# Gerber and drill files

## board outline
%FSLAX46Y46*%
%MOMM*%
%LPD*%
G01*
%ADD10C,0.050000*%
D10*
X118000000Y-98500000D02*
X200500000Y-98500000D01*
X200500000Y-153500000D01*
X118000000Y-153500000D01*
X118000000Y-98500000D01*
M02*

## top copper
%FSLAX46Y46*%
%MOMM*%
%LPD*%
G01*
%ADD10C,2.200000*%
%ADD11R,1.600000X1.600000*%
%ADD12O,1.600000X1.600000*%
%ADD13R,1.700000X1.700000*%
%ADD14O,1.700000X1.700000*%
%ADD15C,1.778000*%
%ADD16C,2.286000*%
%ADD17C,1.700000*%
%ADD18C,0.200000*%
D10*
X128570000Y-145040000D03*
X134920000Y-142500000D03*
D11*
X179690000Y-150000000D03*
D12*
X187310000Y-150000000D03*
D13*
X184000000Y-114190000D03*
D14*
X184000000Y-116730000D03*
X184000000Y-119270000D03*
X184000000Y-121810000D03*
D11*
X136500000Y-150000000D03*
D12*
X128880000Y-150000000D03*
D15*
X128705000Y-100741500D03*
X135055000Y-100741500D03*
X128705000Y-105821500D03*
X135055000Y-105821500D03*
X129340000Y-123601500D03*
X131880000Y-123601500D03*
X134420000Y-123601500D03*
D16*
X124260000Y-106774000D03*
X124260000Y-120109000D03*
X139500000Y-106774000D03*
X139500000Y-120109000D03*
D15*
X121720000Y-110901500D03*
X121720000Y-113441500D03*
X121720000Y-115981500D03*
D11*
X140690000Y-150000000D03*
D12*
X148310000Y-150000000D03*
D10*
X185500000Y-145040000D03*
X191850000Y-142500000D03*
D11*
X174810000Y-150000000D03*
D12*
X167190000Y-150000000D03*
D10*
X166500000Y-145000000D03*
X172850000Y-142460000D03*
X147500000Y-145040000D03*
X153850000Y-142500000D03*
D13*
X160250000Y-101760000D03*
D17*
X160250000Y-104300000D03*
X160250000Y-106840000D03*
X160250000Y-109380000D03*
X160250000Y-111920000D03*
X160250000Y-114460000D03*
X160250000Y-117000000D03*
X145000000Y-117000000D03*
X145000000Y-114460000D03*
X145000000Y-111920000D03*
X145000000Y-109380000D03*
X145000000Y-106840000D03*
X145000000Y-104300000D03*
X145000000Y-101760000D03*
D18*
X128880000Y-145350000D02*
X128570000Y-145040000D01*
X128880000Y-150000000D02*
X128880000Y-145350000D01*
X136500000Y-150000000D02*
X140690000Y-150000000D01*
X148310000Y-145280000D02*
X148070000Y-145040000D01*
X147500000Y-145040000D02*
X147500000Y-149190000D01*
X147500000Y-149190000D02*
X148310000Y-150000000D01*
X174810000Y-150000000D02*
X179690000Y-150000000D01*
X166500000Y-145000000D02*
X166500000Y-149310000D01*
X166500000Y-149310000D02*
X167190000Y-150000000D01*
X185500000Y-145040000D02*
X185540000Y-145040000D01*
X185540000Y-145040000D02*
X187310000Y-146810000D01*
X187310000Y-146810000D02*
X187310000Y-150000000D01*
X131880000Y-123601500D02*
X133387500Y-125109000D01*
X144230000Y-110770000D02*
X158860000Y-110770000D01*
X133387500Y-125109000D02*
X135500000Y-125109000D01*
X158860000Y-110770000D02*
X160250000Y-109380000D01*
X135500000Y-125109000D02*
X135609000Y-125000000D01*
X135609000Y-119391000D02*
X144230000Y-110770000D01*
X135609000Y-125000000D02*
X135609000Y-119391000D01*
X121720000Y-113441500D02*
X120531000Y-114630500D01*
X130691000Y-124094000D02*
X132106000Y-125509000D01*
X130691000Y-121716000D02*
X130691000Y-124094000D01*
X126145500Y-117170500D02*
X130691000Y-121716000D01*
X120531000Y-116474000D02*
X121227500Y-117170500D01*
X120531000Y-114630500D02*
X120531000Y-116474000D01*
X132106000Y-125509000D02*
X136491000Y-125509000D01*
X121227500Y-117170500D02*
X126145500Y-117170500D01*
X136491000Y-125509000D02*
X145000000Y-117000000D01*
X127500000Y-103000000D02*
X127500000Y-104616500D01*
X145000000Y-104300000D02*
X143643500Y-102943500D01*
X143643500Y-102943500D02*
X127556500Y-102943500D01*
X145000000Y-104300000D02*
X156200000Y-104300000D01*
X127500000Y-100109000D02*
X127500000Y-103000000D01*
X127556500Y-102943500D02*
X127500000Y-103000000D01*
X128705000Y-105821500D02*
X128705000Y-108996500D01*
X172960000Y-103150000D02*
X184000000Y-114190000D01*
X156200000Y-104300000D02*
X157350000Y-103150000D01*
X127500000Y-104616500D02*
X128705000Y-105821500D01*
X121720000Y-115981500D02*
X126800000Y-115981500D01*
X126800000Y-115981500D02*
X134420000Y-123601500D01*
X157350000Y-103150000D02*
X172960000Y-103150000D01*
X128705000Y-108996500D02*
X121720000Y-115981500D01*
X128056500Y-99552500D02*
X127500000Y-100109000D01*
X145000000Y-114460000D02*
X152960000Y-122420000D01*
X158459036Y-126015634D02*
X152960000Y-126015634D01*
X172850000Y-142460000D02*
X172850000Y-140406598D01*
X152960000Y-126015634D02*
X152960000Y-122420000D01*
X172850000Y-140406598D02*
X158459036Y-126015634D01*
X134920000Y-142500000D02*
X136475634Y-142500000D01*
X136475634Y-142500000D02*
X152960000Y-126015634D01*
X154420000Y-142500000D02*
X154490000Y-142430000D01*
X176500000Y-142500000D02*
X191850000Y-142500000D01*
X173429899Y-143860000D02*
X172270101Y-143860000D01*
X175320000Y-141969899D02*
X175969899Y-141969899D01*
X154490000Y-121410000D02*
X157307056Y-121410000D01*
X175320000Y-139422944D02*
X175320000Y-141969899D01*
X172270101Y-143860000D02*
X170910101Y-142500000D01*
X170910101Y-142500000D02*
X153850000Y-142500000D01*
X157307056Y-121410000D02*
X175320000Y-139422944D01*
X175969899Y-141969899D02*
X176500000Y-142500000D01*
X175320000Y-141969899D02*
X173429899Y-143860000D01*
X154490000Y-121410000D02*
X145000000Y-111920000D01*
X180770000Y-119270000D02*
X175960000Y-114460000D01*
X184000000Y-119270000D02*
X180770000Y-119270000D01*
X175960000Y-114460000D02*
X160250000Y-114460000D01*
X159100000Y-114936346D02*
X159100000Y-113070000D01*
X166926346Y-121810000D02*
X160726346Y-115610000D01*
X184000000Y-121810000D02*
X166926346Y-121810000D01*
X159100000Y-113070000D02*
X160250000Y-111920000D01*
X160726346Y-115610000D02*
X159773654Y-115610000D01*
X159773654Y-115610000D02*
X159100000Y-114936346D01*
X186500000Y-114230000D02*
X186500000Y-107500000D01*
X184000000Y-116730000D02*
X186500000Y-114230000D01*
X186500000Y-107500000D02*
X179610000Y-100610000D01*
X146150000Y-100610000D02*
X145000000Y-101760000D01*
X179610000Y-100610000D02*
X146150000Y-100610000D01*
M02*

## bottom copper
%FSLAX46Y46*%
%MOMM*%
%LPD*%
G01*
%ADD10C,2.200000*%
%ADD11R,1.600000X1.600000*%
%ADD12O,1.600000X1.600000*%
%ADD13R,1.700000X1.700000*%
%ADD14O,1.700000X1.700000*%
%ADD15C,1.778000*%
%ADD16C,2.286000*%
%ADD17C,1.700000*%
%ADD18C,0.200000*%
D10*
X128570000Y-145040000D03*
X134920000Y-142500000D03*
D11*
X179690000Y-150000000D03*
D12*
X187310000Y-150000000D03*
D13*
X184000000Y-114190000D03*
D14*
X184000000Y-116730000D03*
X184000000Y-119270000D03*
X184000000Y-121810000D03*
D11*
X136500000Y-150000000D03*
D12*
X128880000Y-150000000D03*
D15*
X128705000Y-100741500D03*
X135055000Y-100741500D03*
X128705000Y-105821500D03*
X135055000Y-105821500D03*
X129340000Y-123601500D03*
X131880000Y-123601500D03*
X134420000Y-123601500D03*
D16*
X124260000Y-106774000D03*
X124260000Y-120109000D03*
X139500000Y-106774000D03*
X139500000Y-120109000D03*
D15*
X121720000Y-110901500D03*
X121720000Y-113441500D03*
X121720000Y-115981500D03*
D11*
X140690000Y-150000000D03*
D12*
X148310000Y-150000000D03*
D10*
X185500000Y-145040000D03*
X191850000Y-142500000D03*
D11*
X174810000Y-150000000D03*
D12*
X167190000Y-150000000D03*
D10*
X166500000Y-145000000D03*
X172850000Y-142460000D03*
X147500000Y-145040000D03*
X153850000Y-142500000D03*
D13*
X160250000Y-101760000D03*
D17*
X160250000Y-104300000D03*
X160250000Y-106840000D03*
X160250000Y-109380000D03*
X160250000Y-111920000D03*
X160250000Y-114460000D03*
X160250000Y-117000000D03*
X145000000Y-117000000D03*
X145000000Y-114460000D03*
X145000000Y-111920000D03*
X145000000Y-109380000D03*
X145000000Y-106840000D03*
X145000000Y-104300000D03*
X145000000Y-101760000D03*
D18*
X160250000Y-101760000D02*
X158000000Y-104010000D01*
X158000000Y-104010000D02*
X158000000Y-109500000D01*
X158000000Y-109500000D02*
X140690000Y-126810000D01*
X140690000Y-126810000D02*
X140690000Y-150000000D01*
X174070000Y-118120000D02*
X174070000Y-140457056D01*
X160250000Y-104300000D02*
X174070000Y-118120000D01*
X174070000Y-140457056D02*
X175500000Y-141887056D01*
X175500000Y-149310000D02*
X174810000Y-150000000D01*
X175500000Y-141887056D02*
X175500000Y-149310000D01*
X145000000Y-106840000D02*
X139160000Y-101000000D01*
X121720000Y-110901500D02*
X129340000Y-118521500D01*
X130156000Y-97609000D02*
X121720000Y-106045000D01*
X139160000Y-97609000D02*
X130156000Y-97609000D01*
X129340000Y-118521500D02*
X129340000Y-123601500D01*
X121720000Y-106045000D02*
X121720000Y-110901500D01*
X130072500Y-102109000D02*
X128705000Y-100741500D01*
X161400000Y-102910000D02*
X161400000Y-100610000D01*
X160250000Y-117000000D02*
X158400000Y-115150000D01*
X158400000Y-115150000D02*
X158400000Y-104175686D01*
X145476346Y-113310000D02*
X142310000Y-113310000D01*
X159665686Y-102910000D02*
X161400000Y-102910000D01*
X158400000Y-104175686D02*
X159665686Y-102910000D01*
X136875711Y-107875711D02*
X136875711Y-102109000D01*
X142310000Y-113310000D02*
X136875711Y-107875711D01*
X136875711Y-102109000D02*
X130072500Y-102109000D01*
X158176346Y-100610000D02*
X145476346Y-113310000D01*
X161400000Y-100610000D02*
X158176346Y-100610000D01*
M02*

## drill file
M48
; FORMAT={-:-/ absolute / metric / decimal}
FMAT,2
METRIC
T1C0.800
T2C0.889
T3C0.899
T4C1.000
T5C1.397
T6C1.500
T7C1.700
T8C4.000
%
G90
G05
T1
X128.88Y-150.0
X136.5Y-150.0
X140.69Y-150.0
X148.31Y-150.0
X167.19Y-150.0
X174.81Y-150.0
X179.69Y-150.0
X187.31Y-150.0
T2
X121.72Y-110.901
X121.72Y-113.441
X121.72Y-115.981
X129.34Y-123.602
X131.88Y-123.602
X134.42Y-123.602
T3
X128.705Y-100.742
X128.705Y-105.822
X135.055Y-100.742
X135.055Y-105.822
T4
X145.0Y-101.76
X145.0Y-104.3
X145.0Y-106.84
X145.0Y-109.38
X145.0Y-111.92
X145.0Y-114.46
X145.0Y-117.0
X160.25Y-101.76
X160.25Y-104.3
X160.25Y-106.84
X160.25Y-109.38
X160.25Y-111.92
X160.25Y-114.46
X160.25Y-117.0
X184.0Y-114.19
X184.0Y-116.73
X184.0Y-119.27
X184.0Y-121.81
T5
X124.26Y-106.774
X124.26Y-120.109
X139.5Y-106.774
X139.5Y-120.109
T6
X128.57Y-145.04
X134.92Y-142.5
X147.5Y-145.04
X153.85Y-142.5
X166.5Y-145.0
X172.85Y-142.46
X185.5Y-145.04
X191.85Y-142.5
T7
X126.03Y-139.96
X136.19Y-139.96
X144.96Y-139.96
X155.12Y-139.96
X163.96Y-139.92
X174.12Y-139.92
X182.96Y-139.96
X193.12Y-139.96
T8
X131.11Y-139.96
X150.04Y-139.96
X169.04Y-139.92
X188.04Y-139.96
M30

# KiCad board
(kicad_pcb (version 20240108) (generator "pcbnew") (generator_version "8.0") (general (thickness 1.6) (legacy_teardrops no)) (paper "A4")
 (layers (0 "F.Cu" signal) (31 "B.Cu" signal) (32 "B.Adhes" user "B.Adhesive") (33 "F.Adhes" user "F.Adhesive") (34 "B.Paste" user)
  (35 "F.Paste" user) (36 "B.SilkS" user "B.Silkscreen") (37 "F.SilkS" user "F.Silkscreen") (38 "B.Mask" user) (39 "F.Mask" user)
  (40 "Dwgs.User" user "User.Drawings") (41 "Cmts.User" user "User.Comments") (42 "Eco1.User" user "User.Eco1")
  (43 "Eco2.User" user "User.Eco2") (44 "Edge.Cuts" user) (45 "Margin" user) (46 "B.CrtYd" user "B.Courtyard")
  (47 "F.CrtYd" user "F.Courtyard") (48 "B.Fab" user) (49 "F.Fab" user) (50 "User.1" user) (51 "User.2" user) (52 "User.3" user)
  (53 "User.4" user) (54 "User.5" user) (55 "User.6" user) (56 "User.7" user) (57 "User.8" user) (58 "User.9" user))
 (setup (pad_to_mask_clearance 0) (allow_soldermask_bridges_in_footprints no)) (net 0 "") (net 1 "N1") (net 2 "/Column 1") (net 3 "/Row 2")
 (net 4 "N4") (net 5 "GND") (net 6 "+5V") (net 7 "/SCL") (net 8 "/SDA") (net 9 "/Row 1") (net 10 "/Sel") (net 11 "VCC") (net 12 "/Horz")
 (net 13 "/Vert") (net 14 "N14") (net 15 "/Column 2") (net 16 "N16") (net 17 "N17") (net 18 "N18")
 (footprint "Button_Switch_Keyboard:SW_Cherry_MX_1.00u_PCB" (layer "F.Cu") (at 128.57 145.04 180)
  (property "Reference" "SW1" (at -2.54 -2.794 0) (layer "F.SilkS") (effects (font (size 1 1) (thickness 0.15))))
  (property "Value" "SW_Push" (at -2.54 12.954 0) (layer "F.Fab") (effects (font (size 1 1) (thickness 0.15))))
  (pad "" np_thru_hole circle (at -7.62 5.08 180) (size 1.7 1.7) (drill 1.7) (layers "*.Cu" "*.Mask"))
  (pad "" np_thru_hole circle (at -2.54 5.08 180) (size 4 4) (drill 4) (layers "*.Cu" "*.Mask"))
  (pad "" np_thru_hole circle (at 2.54 5.08 180) (size 1.7 1.7) (drill 1.7) (layers "*.Cu" "*.Mask"))
  (pad "1" thru_hole circle (at 0 0 180) (size 2.2 2.2) (drill 1.5) (layers "*.Cu" "*.Mask") (remove_unused_layers no) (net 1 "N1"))
  (pad "2" thru_hole circle (at -6.35 2.54 180) (size 2.2 2.2) (drill 1.5) (layers "*.Cu" "*.Mask") (remove_unused_layers no)
   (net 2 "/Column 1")))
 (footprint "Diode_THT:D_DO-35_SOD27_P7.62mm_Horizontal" (layer "F.Cu") (at 179.69 150)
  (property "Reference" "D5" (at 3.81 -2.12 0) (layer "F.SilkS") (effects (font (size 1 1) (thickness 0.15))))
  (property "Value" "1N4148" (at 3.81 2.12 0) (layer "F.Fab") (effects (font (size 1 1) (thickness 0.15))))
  (pad "1" thru_hole rect (at 0 0) (size 1.6 1.6) (drill 0.8) (layers "*.Cu" "*.Mask") (remove_unused_layers no) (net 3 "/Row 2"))
  (pad "2" thru_hole oval (at 7.62 0) (size 1.6 1.6) (drill 0.8) (layers "*.Cu" "*.Mask") (remove_unused_layers no) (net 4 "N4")))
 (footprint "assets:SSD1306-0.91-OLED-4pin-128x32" (layer "F.Cu") (at 147.5 112)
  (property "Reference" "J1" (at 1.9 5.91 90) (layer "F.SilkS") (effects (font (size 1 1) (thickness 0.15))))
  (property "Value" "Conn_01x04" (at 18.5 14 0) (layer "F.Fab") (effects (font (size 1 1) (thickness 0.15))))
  (pad "1" thru_hole rect (at 36.5 2.19) (size 1.7 1.7) (drill 1) (layers "*.Cu" "*.Mask") (remove_unused_layers no) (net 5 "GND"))
  (pad "2" thru_hole oval (at 36.5 4.73) (size 1.7 1.7) (drill 1) (layers "*.Cu" "*.Mask") (remove_unused_layers no) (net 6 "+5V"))
  (pad "3" thru_hole oval (at 36.5 7.27) (size 1.7 1.7) (drill 1) (layers "*.Cu" "*.Mask") (remove_unused_layers no) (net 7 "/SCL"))
  (pad "4" thru_hole oval (at 36.5 9.81) (size 1.7 1.7) (drill 1) (layers "*.Cu" "*.Mask") (remove_unused_layers no) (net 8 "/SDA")))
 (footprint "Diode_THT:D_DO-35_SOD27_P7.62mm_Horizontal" (layer "F.Cu") (at 136.5 150 180)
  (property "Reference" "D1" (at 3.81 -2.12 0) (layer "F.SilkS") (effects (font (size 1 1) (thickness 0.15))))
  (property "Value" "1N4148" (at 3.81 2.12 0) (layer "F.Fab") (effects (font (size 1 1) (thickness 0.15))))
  (pad "1" thru_hole rect (at 0 0 180) (size 1.6 1.6) (drill 0.8) (layers "*.Cu" "*.Mask") (remove_unused_layers no) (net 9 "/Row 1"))
  (pad "2" thru_hole oval (at 7.62 0 180) (size 1.6 1.6) (drill 0.8) (layers "*.Cu" "*.Mask") (remove_unused_layers no) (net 1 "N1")))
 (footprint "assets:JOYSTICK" (layer "F.Cu") (at 131.88 113.4415)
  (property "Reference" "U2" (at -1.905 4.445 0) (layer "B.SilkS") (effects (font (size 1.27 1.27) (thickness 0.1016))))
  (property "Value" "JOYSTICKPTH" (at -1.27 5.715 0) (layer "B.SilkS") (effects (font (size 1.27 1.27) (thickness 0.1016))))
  (pad "B1A" thru_hole circle (at -3.175 -12.7) (size 1.778 1.778) (drill 0.89916) (layers "F&B.Cu" "F.Paste" "F.SilkS" "F.Mask")
   (remove_unused_layers no) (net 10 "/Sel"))
  (pad "B1B" thru_hole circle (at 3.175 -12.7) (size 1.778 1.778) (drill 0.89916) (layers "F&B.Cu" "F.Paste" "F.SilkS" "F.Mask")
   (remove_unused_layers no))
  (pad "B2A" thru_hole circle (at -3.175 -7.62) (size 1.778 1.778) (drill 0.89916) (layers "F&B.Cu" "F.Paste" "F.SilkS" "F.Mask")
   (remove_unused_layers no) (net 5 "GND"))
  (pad "B2B" thru_hole circle (at 3.175 -7.62) (size 1.778 1.778) (drill 0.89916) (layers "F&B.Cu" "F.Paste" "F.SilkS" "F.Mask")
   (remove_unused_layers no))
  (pad "H1" thru_hole circle (at -2.54 10.16) (size 1.778 1.778) (drill 0.889) (layers "F&B.Cu" "F.Paste" "F.SilkS" "F.Mask")
   (remove_unused_layers no) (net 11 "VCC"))
  (pad "H2" thru_hole circle (at 0 10.16) (size 1.778 1.778) (drill 0.889) (layers "F&B.Cu" "F.Paste" "F.SilkS" "F.Mask")
   (remove_unused_layers no) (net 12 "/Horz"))
  (pad "H3" thru_hole circle (at 2.54 10.16) (size 1.778 1.778) (drill 0.889) (layers "F&B.Cu" "F.Paste" "F.SilkS" "F.Mask")
   (remove_unused_layers no) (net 5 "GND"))
  (pad "MOUN" thru_hole circle (at -7.62 -6.6675) (size 2.286 2.286) (drill 1.397) (layers "F&B.Cu" "F.Paste" "F.SilkS" "F.Mask")
   (remove_unused_layers no))
  (pad "MOUN" thru_hole circle (at -7.62 6.6675) (size 2.286 2.286) (drill 1.397) (layers "F&B.Cu" "F.Paste" "F.SilkS" "F.Mask")
   (remove_unused_layers no))
  (pad "MOUN" thru_hole circle (at 7.62 -6.6675) (size 2.286 2.286) (drill 1.397) (layers "F&B.Cu" "F.Paste" "F.SilkS" "F.Mask")
   (remove_unused_layers no))
  (pad "MOUN" thru_hole circle (at 7.62 6.6675) (size 2.286 2.286) (drill 1.397) (layers "F&B.Cu" "F.Paste" "F.SilkS" "F.Mask")
   (remove_unused_layers no))
  (pad "V1" thru_hole circle (at -10.16 -2.54) (size 1.778 1.778) (drill 0.889) (layers "F&B.Cu" "F.Paste" "F.SilkS" "F.Mask")
   (remove_unused_layers no) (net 11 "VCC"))
  (pad "V2" thru_hole circle (at -10.16 0) (size 1.778 1.778) (drill 0.889) (layers "F&B.Cu" "F.Paste" "F.SilkS" "F.Mask")
   (remove_unused_layers no) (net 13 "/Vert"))
  (pad "V3" thru_hole circle (at -10.16 2.54) (size 1.778 1.778) (drill 0.889) (layers "F&B.Cu" "F.Paste" "F.SilkS" "F.Mask")
   (remove_unused_layers no) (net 5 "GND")))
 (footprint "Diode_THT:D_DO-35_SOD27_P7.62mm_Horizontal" (layer "F.Cu") (at 140.69 150)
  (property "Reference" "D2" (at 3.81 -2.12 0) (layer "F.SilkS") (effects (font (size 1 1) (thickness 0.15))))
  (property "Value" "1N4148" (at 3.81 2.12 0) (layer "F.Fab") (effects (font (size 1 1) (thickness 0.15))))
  (pad "1" thru_hole rect (at 0 0) (size 1.6 1.6) (drill 0.8) (layers "*.Cu" "*.Mask") (remove_unused_layers no) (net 9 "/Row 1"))
  (pad "2" thru_hole oval (at 7.62 0) (size 1.6 1.6) (drill 0.8) (layers "*.Cu" "*.Mask") (remove_unused_layers no) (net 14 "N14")))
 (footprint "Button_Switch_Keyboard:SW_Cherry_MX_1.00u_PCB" (layer "F.Cu") (at 185.5 145.04 180)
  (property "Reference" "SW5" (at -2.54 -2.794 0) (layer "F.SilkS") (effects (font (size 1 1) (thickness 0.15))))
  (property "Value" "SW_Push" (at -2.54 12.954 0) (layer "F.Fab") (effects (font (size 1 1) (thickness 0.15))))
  (pad "" np_thru_hole circle (at -7.62 5.08 180) (size 1.7 1.7) (drill 1.7) (layers "*.Cu" "*.Mask"))
  (pad "" np_thru_hole circle (at -2.54 5.08 180) (size 4 4) (drill 4) (layers "*.Cu" "*.Mask"))
  (pad "" np_thru_hole circle (at 2.54 5.08 180) (size 1.7 1.7) (drill 1.7) (layers "*.Cu" "*.Mask"))
  (pad "1" thru_hole circle (at 0 0 180) (size 2.2 2.2) (drill 1.5) (layers "*.Cu" "*.Mask") (remove_unused_layers no) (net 4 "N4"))
  (pad "2" thru_hole circle (at -6.35 2.54 180) (size 2.2 2.2) (drill 1.5) (layers "*.Cu" "*.Mask") (remove_unused_layers no)
   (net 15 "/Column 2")))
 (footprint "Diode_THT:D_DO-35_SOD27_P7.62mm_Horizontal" (layer "F.Cu") (at 174.81 150 180)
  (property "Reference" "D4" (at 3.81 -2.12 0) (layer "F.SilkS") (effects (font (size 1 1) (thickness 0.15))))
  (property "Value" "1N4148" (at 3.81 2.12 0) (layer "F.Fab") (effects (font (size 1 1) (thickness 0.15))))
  (pad "1" thru_hole rect (at 0 0 180) (size 1.6 1.6) (drill 0.8) (layers "*.Cu" "*.Mask") (remove_unused_layers no) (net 3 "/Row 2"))
  (pad "2" thru_hole oval (at 7.62 0 180) (size 1.6 1.6) (drill 0.8) (layers "*.Cu" "*.Mask") (remove_unused_layers no) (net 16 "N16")))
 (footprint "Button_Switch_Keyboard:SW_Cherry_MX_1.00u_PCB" (layer "F.Cu") (at 166.5 145 180)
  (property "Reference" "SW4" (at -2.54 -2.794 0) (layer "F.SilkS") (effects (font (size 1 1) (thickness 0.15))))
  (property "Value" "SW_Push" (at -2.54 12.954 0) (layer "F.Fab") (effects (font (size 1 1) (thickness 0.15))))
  (pad "" np_thru_hole circle (at -7.62 5.08 180) (size 1.7 1.7) (drill 1.7) (layers "*.Cu" "*.Mask"))
  (pad "" np_thru_hole circle (at -2.54 5.08 180) (size 4 4) (drill 4) (layers "*.Cu" "*.Mask"))
  (pad "" np_thru_hole circle (at 2.54 5.08 180) (size 1.7 1.7) (drill 1.7) (layers "*.Cu" "*.Mask"))
  (pad "1" thru_hole circle (at 0 0 180) (size 2.2 2.2) (drill 1.5) (layers "*.Cu" "*.Mask") (remove_unused_layers no) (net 16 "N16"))
  (pad "2" thru_hole circle (at -6.35 2.54 180) (size 2.2 2.2) (drill 1.5) (layers "*.Cu" "*.Mask") (remove_unused_layers no)
   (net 2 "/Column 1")))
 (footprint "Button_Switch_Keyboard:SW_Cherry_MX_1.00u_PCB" (layer "F.Cu") (at 147.5 145.04 180)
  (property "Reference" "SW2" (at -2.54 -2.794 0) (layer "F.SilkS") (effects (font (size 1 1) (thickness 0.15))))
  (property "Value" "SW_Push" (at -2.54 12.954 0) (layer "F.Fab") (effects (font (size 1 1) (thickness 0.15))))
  (pad "" np_thru_hole circle (at -7.62 5.08 180) (size 1.7 1.7) (drill 1.7) (layers "*.Cu" "*.Mask"))
  (pad "" np_thru_hole circle (at -2.54 5.08 180) (size 4 4) (drill 4) (layers "*.Cu" "*.Mask"))
  (pad "" np_thru_hole circle (at 2.54 5.08 180) (size 1.7 1.7) (drill 1.7) (layers "*.Cu" "*.Mask"))
  (pad "1" thru_hole circle (at 0 0 180) (size 2.2 2.2) (drill 1.5) (layers "*.Cu" "*.Mask") (remove_unused_layers no) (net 14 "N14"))
  (pad "2" thru_hole circle (at -6.35 2.54 180) (size 2.2 2.2) (drill 1.5) (layers "*.Cu" "*.Mask") (remove_unused_layers no)
   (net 15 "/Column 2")))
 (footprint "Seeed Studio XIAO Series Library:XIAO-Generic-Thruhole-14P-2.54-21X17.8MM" (layer "B.Cu") (at 152.625 109.38 180)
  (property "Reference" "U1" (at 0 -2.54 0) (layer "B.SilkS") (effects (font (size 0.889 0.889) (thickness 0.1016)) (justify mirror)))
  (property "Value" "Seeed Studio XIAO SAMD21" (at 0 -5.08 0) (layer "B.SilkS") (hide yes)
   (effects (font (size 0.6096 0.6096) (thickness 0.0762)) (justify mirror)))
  (pad "1" thru_hole rect (at -7.625 7.62 180) (size 1.7 1.7) (drill 1) (layers "*.Cu" "*.Mask") (remove_unused_layers no) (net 9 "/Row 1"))
  (pad "2" thru_hole circle (at -7.625 5.08 180) (size 1.7 1.7) (drill 1) (layers "*.Cu" "*.Mask") (remove_unused_layers no)
   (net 3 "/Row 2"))
  (pad "3" thru_hole circle (at -7.625 2.54 180) (size 1.7 1.7) (drill 1) (layers "*.Cu" "*.Mask") (remove_unused_layers no) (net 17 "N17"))
  (pad "4" thru_hole circle (at -7.625 0 180) (size 1.7 1.7) (drill 1) (layers "*.Cu" "*.Mask") (remove_unused_layers no) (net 12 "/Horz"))
  (pad "5" thru_hole circle (at -7.625 -2.54 180) (size 1.7 1.7) (drill 1) (layers "*.Cu" "*.Mask") (remove_unused_layers no) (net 8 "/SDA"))
  (pad "6" thru_hole circle (at -7.625 -5.08) (size 1.7 1.7) (drill 1) (layers "*.Cu" "*.Mask") (remove_unused_layers no) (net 7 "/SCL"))
  (pad "7" thru_hole circle (at -7.625 -7.62 180) (size 1.7 1.7) (drill 1) (layers "*.Cu" "*.Mask") (remove_unused_layers no)
   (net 10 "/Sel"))
  (pad "8" thru_hole circle (at 7.625 -7.62 180) (size 1.7 1.7) (drill 1) (layers "*.Cu" "*.Mask") (remove_unused_layers no)
   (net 13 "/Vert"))
  (pad "9" thru_hole circle (at 7.625 -5.08 180) (size 1.7 1.7) (drill 1) (layers "*.Cu" "*.Mask") (remove_unused_layers no)
   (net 2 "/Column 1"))
  (pad "10" thru_hole circle (at 7.625 -2.54 180) (size 1.7 1.7) (drill 1) (layers "*.Cu" "*.Mask") (remove_unused_layers no)
   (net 15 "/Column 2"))
  (pad "11" thru_hole circle (at 7.625 0 180) (size 1.7 1.7) (drill 1) (layers "*.Cu" "*.Mask") (remove_unused_layers no) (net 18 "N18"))
  (pad "12" thru_hole circle (at 7.625 2.54 180) (size 1.7 1.7) (drill 1) (layers "*.Cu" "*.Mask") (remove_unused_layers no) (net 11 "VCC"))
  (pad "13" thru_hole circle (at 7.625 5.08 180) (size 1.7 1.7) (drill 1) (layers "*.Cu" "*.Mask") (remove_unused_layers no) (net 5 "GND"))
  (pad "14" thru_hole circle (at 7.625 7.62 180) (size 1.7 1.7) (drill 1) (layers "*.Cu" "*.Mask") (remove_unused_layers no) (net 6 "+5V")))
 (gr_rect (start 118 98.5) (end 200.5 153.5) (stroke (width 0.05) (type default)) (fill none) (layer "Edge.Cuts"))
 (segment (start 128.88 145.35) (end 128.57 145.04) (width 0.2) (layer "F.Cu") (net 1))
 (segment (start 128.88 150) (end 128.88 145.35) (width 0.2) (layer "F.Cu") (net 1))
 (segment (start 136.5 150) (end 140.69 150) (width 0.2) (layer "F.Cu") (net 9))
 (segment (start 160.25 101.76) (end 158 104.01) (width 0.2) (layer "B.Cu") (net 9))
 (segment (start 158 104.01) (end 158 109.5) (width 0.2) (layer "B.Cu") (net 9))
 (segment (start 158 109.5) (end 140.69 126.81) (width 0.2) (layer "B.Cu") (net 9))
 (segment (start 140.69 126.81) (end 140.69 150) (width 0.2) (layer "B.Cu") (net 9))
 (segment (start 148.31 145.28) (end 148.07 145.04) (width 0.2) (layer "F.Cu") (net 14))
 (segment (start 147.5 145.04) (end 147.5 149.19) (width 0.2) (layer "F.Cu") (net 14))
 (segment (start 147.5 149.19) (end 148.31 150) (width 0.2) (layer "F.Cu") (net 14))
 (segment (start 174.81 150) (end 179.69 150) (width 0.2) (layer "F.Cu") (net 3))
 (segment (start 174.07 118.12) (end 174.07 140.457056) (width 0.2) (layer "B.Cu") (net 3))
 (segment (start 160.25 104.3) (end 174.07 118.12) (width 0.2) (layer "B.Cu") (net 3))
 (segment (start 174.07 140.457056) (end 175.5 141.887056) (width 0.2) (layer "B.Cu") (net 3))
 (segment (start 175.5 149.31) (end 174.81 150) (width 0.2) (layer "B.Cu") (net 3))
 (segment (start 175.5 141.887056) (end 175.5 149.31) (width 0.2) (layer "B.Cu") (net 3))
 (segment (start 166.5 145) (end 166.5 149.31) (width 0.2) (layer "F.Cu") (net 16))
 (segment (start 166.5 149.31) (end 167.19 150) (width 0.2) (layer "F.Cu") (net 16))
 (segment (start 185.5 145.04) (end 185.54 145.04) (width 0.2) (layer "F.Cu") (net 4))
 (segment (start 185.54 145.04) (end 187.31 146.81) (width 0.2) (layer "F.Cu") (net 4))
 (segment (start 187.31 146.81) (end 187.31 150) (width 0.2) (layer "F.Cu") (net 4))
 (segment (start 131.88 123.6015) (end 133.3875 125.109) (width 0.2) (layer "F.Cu") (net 12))
 (segment (start 144.23 110.77) (end 158.86 110.77) (width 0.2) (layer "F.Cu") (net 12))
 (segment (start 133.3875 125.109) (end 135.5 125.109) (width 0.2) (layer "F.Cu") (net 12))
 (segment (start 158.86 110.77) (end 160.25 109.38) (width 0.2) (layer "F.Cu") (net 12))
 (segment (start 135.5 125.109) (end 135.609 125) (width 0.2) (layer "F.Cu") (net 12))
 (segment (start 135.609 119.391) (end 144.23 110.77) (width 0.2) (layer "F.Cu") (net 12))
 (segment (start 135.609 125) (end 135.609 119.391) (width 0.2) (layer "F.Cu") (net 12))
 (segment (start 145 106.84) (end 139.16 101) (width 0.2) (layer "B.Cu") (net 11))
 (segment (start 121.72 110.9015) (end 129.34 118.5215) (width 0.2) (layer "B.Cu") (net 11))
 (segment (start 130.156 97.609) (end 121.72 106.045) (width 0.2) (layer "B.Cu") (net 11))
 (segment (start 139.16 97.609) (end 130.156 97.609) (width 0.2) (layer "B.Cu") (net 11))
 (segment (start 129.34 118.5215) (end 129.34 123.6015) (width 0.2) (layer "B.Cu") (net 11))
 (segment (start 121.72 106.045) (end 121.72 110.9015) (width 0.2) (layer "B.Cu") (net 11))
 (segment (start 121.72 113.4415) (end 120.531 114.6305) (width 0.2) (layer "F.Cu") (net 13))
 (segment (start 130.691 124.094) (end 132.106 125.509) (width 0.2) (layer "F.Cu") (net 13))
 (segment (start 130.691 121.716) (end 130.691 124.094) (width 0.2) (layer "F.Cu") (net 13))
 (segment (start 126.1455 117.1705) (end 130.691 121.716) (width 0.2) (layer "F.Cu") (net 13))
 (segment (start 120.531 116.474) (end 121.2275 117.1705) (width 0.2) (layer "F.Cu") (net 13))
 (segment (start 120.531 114.6305) (end 120.531 116.474) (width 0.2) (layer "F.Cu") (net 13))
 (segment (start 132.106 125.509) (end 136.491 125.509) (width 0.2) (layer "F.Cu") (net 13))
 (segment (start 121.2275 117.1705) (end 126.1455 117.1705) (width 0.2) (layer "F.Cu") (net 13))
 (segment (start 136.491 125.509) (end 145 117) (width 0.2) (layer "F.Cu") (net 13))
 (segment (start 130.0725 102.109) (end 128.705 100.7415) (width 0.2) (layer "B.Cu") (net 10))
 (segment (start 161.4 102.91) (end 161.4 100.61) (width 0.2) (layer "B.Cu") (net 10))
 (segment (start 160.25 117) (end 158.4 115.15) (width 0.2) (layer "B.Cu") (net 10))
 (segment (start 158.4 115.15) (end 158.4 104.175686) (width 0.2) (layer "B.Cu") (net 10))
 (segment (start 145.476346 113.31) (end 142.31 113.31) (width 0.2) (layer "B.Cu") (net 10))
 (segment (start 159.665686 102.91) (end 161.4 102.91) (width 0.2) (layer "B.Cu") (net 10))
 (segment (start 158.4 104.175686) (end 159.665686 102.91) (width 0.2) (layer "B.Cu") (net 10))
 (segment (start 136.875711 107.875711) (end 136.875711 102.109) (width 0.2) (layer "B.Cu") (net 10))
 (segment (start 142.31 113.31) (end 136.875711 107.875711) (width 0.2) (layer "B.Cu") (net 10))
 (segment (start 136.875711 102.109) (end 130.0725 102.109) (width 0.2) (layer "B.Cu") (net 10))
 (segment (start 158.176346 100.61) (end 145.476346 113.31) (width 0.2) (layer "B.Cu") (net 10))
 (segment (start 161.4 100.61) (end 158.176346 100.61) (width 0.2) (layer "B.Cu") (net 10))
 (segment (start 127.5 103) (end 127.5 104.6165) (width 0.2) (layer "F.Cu") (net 5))
 (segment (start 145 104.3) (end 143.6435 102.9435) (width 0.2) (layer "F.Cu") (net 5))
 (segment (start 143.6435 102.9435) (end 127.5565 102.9435) (width 0.2) (layer "F.Cu") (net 5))
 (segment (start 145 104.3) (end 156.2 104.3) (width 0.2) (layer "F.Cu") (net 5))
 (segment (start 127.5 100.109) (end 127.5 103) (width 0.2) (layer "F.Cu") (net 5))
 (segment (start 127.5565 102.9435) (end 127.5 103) (width 0.2) (layer "F.Cu") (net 5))
 (segment (start 128.705 105.8215) (end 128.705 108.9965) (width 0.2) (layer "F.Cu") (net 5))
 (segment (start 172.96 103.15) (end 184 114.19) (width 0.2) (layer "F.Cu") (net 5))
 (segment (start 156.2 104.3) (end 157.35 103.15) (width 0.2) (layer "F.Cu") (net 5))
 (segment (start 127.5 104.6165) (end 128.705 105.8215) (width 0.2) (layer "F.Cu") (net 5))
 (segment (start 121.72 115.9815) (end 126.8 115.9815) (width 0.2) (layer "F.Cu") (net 5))
 (segment (start 126.8 115.9815) (end 134.42 123.6015) (width 0.2) (layer "F.Cu") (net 5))
 (segment (start 157.35 103.15) (end 172.96 103.15) (width 0.2) (layer "F.Cu") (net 5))
 (segment (start 128.705 108.9965) (end 121.72 115.9815) (width 0.2) (layer "F.Cu") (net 5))
 (segment (start 128.0565 99.5525) (end 127.5 100.109) (width 0.2) (layer "F.Cu") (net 5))
 (segment (start 145 114.46) (end 152.96 122.42) (width 0.2) (layer "F.Cu") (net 2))
 (segment (start 158.459036 126.015634) (end 152.96 126.015634) (width 0.2) (layer "F.Cu") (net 2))
 (segment (start 172.85 142.46) (end 172.85 140.406598) (width 0.2) (layer "F.Cu") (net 2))
 (segment (start 152.96 126.015634) (end 152.96 122.42) (width 0.2) (layer "F.Cu") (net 2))
 (segment (start 172.85 140.406598) (end 158.459036 126.015634) (width 0.2) (layer "F.Cu") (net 2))
 (segment (start 134.92 142.5) (end 136.475634 142.5) (width 0.2) (layer "F.Cu") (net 2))
 (segment (start 136.475634 142.5) (end 152.96 126.015634) (width 0.2) (layer "F.Cu") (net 2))
 (segment (start 154.42 142.5) (end 154.49 142.43) (width 0.2) (layer "F.Cu") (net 15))
 (segment (start 176.5 142.5) (end 191.85 142.5) (width 0.2) (layer "F.Cu") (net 15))
 (segment (start 173.429899 143.86) (end 172.270101 143.86) (width 0.2) (layer "F.Cu") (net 15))
 (segment (start 175.32 141.969899) (end 175.969899 141.969899) (width 0.2) (layer "F.Cu") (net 15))
 (segment (start 154.49 121.41) (end 157.307056 121.41) (width 0.2) (layer "F.Cu") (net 15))
 (segment (start 175.32 139.422944) (end 175.32 141.969899) (width 0.2) (layer "F.Cu") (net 15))
 (segment (start 172.270101 143.86) (end 170.910101 142.5) (width 0.2) (layer "F.Cu") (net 15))
 (segment (start 170.910101 142.5) (end 153.85 142.5) (width 0.2) (layer "F.Cu") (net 15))
 (segment (start 157.307056 121.41) (end 175.32 139.422944) (width 0.2) (layer "F.Cu") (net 15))
 (segment (start 175.969899 141.969899) (end 176.5 142.5) (width 0.2) (layer "F.Cu") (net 15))
 (segment (start 175.32 141.969899) (end 173.429899 143.86) (width 0.2) (layer "F.Cu") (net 15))
 (segment (start 154.49 121.41) (end 145 111.92) (width 0.2) (layer "F.Cu") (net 15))
 (segment (start 180.77 119.27) (end 175.96 114.46) (width 0.2) (layer "F.Cu") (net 7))
 (segment (start 184 119.27) (end 180.77 119.27) (width 0.2) (layer "F.Cu") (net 7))
 (segment (start 175.96 114.46) (end 160.25 114.46) (width 0.2) (layer "F.Cu") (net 7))
 (segment (start 159.1 114.936346) (end 159.1 113.07) (width 0.2) (layer "F.Cu") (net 8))
 (segment (start 166.926346 121.81) (end 160.726346 115.61) (width 0.2) (layer "F.Cu") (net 8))
 (segment (start 184 121.81) (end 166.926346 121.81) (width 0.2) (layer "F.Cu") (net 8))
 (segment (start 159.1 113.07) (end 160.25 111.92) (width 0.2) (layer "F.Cu") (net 8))
 (segment (start 160.726346 115.61) (end 159.773654 115.61) (width 0.2) (layer "F.Cu") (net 8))
 (segment (start 159.773654 115.61) (end 159.1 114.936346) (width 0.2) (layer "F.Cu") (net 8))
 (segment (start 186.5 114.23) (end 186.5 107.5) (width 0.2) (layer "F.Cu") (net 6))
 (segment (start 184 116.73) (end 186.5 114.23) (width 0.2) (layer "F.Cu") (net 6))
 (segment (start 186.5 107.5) (end 179.61 100.61) (width 0.2) (layer "F.Cu") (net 6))
 (segment (start 146.15 100.61) (end 145 101.76) (width 0.2) (layer "F.Cu") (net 6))
 (segment (start 179.61 100.61) (end 146.15 100.61) (width 0.2) (layer "F.Cu") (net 6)))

